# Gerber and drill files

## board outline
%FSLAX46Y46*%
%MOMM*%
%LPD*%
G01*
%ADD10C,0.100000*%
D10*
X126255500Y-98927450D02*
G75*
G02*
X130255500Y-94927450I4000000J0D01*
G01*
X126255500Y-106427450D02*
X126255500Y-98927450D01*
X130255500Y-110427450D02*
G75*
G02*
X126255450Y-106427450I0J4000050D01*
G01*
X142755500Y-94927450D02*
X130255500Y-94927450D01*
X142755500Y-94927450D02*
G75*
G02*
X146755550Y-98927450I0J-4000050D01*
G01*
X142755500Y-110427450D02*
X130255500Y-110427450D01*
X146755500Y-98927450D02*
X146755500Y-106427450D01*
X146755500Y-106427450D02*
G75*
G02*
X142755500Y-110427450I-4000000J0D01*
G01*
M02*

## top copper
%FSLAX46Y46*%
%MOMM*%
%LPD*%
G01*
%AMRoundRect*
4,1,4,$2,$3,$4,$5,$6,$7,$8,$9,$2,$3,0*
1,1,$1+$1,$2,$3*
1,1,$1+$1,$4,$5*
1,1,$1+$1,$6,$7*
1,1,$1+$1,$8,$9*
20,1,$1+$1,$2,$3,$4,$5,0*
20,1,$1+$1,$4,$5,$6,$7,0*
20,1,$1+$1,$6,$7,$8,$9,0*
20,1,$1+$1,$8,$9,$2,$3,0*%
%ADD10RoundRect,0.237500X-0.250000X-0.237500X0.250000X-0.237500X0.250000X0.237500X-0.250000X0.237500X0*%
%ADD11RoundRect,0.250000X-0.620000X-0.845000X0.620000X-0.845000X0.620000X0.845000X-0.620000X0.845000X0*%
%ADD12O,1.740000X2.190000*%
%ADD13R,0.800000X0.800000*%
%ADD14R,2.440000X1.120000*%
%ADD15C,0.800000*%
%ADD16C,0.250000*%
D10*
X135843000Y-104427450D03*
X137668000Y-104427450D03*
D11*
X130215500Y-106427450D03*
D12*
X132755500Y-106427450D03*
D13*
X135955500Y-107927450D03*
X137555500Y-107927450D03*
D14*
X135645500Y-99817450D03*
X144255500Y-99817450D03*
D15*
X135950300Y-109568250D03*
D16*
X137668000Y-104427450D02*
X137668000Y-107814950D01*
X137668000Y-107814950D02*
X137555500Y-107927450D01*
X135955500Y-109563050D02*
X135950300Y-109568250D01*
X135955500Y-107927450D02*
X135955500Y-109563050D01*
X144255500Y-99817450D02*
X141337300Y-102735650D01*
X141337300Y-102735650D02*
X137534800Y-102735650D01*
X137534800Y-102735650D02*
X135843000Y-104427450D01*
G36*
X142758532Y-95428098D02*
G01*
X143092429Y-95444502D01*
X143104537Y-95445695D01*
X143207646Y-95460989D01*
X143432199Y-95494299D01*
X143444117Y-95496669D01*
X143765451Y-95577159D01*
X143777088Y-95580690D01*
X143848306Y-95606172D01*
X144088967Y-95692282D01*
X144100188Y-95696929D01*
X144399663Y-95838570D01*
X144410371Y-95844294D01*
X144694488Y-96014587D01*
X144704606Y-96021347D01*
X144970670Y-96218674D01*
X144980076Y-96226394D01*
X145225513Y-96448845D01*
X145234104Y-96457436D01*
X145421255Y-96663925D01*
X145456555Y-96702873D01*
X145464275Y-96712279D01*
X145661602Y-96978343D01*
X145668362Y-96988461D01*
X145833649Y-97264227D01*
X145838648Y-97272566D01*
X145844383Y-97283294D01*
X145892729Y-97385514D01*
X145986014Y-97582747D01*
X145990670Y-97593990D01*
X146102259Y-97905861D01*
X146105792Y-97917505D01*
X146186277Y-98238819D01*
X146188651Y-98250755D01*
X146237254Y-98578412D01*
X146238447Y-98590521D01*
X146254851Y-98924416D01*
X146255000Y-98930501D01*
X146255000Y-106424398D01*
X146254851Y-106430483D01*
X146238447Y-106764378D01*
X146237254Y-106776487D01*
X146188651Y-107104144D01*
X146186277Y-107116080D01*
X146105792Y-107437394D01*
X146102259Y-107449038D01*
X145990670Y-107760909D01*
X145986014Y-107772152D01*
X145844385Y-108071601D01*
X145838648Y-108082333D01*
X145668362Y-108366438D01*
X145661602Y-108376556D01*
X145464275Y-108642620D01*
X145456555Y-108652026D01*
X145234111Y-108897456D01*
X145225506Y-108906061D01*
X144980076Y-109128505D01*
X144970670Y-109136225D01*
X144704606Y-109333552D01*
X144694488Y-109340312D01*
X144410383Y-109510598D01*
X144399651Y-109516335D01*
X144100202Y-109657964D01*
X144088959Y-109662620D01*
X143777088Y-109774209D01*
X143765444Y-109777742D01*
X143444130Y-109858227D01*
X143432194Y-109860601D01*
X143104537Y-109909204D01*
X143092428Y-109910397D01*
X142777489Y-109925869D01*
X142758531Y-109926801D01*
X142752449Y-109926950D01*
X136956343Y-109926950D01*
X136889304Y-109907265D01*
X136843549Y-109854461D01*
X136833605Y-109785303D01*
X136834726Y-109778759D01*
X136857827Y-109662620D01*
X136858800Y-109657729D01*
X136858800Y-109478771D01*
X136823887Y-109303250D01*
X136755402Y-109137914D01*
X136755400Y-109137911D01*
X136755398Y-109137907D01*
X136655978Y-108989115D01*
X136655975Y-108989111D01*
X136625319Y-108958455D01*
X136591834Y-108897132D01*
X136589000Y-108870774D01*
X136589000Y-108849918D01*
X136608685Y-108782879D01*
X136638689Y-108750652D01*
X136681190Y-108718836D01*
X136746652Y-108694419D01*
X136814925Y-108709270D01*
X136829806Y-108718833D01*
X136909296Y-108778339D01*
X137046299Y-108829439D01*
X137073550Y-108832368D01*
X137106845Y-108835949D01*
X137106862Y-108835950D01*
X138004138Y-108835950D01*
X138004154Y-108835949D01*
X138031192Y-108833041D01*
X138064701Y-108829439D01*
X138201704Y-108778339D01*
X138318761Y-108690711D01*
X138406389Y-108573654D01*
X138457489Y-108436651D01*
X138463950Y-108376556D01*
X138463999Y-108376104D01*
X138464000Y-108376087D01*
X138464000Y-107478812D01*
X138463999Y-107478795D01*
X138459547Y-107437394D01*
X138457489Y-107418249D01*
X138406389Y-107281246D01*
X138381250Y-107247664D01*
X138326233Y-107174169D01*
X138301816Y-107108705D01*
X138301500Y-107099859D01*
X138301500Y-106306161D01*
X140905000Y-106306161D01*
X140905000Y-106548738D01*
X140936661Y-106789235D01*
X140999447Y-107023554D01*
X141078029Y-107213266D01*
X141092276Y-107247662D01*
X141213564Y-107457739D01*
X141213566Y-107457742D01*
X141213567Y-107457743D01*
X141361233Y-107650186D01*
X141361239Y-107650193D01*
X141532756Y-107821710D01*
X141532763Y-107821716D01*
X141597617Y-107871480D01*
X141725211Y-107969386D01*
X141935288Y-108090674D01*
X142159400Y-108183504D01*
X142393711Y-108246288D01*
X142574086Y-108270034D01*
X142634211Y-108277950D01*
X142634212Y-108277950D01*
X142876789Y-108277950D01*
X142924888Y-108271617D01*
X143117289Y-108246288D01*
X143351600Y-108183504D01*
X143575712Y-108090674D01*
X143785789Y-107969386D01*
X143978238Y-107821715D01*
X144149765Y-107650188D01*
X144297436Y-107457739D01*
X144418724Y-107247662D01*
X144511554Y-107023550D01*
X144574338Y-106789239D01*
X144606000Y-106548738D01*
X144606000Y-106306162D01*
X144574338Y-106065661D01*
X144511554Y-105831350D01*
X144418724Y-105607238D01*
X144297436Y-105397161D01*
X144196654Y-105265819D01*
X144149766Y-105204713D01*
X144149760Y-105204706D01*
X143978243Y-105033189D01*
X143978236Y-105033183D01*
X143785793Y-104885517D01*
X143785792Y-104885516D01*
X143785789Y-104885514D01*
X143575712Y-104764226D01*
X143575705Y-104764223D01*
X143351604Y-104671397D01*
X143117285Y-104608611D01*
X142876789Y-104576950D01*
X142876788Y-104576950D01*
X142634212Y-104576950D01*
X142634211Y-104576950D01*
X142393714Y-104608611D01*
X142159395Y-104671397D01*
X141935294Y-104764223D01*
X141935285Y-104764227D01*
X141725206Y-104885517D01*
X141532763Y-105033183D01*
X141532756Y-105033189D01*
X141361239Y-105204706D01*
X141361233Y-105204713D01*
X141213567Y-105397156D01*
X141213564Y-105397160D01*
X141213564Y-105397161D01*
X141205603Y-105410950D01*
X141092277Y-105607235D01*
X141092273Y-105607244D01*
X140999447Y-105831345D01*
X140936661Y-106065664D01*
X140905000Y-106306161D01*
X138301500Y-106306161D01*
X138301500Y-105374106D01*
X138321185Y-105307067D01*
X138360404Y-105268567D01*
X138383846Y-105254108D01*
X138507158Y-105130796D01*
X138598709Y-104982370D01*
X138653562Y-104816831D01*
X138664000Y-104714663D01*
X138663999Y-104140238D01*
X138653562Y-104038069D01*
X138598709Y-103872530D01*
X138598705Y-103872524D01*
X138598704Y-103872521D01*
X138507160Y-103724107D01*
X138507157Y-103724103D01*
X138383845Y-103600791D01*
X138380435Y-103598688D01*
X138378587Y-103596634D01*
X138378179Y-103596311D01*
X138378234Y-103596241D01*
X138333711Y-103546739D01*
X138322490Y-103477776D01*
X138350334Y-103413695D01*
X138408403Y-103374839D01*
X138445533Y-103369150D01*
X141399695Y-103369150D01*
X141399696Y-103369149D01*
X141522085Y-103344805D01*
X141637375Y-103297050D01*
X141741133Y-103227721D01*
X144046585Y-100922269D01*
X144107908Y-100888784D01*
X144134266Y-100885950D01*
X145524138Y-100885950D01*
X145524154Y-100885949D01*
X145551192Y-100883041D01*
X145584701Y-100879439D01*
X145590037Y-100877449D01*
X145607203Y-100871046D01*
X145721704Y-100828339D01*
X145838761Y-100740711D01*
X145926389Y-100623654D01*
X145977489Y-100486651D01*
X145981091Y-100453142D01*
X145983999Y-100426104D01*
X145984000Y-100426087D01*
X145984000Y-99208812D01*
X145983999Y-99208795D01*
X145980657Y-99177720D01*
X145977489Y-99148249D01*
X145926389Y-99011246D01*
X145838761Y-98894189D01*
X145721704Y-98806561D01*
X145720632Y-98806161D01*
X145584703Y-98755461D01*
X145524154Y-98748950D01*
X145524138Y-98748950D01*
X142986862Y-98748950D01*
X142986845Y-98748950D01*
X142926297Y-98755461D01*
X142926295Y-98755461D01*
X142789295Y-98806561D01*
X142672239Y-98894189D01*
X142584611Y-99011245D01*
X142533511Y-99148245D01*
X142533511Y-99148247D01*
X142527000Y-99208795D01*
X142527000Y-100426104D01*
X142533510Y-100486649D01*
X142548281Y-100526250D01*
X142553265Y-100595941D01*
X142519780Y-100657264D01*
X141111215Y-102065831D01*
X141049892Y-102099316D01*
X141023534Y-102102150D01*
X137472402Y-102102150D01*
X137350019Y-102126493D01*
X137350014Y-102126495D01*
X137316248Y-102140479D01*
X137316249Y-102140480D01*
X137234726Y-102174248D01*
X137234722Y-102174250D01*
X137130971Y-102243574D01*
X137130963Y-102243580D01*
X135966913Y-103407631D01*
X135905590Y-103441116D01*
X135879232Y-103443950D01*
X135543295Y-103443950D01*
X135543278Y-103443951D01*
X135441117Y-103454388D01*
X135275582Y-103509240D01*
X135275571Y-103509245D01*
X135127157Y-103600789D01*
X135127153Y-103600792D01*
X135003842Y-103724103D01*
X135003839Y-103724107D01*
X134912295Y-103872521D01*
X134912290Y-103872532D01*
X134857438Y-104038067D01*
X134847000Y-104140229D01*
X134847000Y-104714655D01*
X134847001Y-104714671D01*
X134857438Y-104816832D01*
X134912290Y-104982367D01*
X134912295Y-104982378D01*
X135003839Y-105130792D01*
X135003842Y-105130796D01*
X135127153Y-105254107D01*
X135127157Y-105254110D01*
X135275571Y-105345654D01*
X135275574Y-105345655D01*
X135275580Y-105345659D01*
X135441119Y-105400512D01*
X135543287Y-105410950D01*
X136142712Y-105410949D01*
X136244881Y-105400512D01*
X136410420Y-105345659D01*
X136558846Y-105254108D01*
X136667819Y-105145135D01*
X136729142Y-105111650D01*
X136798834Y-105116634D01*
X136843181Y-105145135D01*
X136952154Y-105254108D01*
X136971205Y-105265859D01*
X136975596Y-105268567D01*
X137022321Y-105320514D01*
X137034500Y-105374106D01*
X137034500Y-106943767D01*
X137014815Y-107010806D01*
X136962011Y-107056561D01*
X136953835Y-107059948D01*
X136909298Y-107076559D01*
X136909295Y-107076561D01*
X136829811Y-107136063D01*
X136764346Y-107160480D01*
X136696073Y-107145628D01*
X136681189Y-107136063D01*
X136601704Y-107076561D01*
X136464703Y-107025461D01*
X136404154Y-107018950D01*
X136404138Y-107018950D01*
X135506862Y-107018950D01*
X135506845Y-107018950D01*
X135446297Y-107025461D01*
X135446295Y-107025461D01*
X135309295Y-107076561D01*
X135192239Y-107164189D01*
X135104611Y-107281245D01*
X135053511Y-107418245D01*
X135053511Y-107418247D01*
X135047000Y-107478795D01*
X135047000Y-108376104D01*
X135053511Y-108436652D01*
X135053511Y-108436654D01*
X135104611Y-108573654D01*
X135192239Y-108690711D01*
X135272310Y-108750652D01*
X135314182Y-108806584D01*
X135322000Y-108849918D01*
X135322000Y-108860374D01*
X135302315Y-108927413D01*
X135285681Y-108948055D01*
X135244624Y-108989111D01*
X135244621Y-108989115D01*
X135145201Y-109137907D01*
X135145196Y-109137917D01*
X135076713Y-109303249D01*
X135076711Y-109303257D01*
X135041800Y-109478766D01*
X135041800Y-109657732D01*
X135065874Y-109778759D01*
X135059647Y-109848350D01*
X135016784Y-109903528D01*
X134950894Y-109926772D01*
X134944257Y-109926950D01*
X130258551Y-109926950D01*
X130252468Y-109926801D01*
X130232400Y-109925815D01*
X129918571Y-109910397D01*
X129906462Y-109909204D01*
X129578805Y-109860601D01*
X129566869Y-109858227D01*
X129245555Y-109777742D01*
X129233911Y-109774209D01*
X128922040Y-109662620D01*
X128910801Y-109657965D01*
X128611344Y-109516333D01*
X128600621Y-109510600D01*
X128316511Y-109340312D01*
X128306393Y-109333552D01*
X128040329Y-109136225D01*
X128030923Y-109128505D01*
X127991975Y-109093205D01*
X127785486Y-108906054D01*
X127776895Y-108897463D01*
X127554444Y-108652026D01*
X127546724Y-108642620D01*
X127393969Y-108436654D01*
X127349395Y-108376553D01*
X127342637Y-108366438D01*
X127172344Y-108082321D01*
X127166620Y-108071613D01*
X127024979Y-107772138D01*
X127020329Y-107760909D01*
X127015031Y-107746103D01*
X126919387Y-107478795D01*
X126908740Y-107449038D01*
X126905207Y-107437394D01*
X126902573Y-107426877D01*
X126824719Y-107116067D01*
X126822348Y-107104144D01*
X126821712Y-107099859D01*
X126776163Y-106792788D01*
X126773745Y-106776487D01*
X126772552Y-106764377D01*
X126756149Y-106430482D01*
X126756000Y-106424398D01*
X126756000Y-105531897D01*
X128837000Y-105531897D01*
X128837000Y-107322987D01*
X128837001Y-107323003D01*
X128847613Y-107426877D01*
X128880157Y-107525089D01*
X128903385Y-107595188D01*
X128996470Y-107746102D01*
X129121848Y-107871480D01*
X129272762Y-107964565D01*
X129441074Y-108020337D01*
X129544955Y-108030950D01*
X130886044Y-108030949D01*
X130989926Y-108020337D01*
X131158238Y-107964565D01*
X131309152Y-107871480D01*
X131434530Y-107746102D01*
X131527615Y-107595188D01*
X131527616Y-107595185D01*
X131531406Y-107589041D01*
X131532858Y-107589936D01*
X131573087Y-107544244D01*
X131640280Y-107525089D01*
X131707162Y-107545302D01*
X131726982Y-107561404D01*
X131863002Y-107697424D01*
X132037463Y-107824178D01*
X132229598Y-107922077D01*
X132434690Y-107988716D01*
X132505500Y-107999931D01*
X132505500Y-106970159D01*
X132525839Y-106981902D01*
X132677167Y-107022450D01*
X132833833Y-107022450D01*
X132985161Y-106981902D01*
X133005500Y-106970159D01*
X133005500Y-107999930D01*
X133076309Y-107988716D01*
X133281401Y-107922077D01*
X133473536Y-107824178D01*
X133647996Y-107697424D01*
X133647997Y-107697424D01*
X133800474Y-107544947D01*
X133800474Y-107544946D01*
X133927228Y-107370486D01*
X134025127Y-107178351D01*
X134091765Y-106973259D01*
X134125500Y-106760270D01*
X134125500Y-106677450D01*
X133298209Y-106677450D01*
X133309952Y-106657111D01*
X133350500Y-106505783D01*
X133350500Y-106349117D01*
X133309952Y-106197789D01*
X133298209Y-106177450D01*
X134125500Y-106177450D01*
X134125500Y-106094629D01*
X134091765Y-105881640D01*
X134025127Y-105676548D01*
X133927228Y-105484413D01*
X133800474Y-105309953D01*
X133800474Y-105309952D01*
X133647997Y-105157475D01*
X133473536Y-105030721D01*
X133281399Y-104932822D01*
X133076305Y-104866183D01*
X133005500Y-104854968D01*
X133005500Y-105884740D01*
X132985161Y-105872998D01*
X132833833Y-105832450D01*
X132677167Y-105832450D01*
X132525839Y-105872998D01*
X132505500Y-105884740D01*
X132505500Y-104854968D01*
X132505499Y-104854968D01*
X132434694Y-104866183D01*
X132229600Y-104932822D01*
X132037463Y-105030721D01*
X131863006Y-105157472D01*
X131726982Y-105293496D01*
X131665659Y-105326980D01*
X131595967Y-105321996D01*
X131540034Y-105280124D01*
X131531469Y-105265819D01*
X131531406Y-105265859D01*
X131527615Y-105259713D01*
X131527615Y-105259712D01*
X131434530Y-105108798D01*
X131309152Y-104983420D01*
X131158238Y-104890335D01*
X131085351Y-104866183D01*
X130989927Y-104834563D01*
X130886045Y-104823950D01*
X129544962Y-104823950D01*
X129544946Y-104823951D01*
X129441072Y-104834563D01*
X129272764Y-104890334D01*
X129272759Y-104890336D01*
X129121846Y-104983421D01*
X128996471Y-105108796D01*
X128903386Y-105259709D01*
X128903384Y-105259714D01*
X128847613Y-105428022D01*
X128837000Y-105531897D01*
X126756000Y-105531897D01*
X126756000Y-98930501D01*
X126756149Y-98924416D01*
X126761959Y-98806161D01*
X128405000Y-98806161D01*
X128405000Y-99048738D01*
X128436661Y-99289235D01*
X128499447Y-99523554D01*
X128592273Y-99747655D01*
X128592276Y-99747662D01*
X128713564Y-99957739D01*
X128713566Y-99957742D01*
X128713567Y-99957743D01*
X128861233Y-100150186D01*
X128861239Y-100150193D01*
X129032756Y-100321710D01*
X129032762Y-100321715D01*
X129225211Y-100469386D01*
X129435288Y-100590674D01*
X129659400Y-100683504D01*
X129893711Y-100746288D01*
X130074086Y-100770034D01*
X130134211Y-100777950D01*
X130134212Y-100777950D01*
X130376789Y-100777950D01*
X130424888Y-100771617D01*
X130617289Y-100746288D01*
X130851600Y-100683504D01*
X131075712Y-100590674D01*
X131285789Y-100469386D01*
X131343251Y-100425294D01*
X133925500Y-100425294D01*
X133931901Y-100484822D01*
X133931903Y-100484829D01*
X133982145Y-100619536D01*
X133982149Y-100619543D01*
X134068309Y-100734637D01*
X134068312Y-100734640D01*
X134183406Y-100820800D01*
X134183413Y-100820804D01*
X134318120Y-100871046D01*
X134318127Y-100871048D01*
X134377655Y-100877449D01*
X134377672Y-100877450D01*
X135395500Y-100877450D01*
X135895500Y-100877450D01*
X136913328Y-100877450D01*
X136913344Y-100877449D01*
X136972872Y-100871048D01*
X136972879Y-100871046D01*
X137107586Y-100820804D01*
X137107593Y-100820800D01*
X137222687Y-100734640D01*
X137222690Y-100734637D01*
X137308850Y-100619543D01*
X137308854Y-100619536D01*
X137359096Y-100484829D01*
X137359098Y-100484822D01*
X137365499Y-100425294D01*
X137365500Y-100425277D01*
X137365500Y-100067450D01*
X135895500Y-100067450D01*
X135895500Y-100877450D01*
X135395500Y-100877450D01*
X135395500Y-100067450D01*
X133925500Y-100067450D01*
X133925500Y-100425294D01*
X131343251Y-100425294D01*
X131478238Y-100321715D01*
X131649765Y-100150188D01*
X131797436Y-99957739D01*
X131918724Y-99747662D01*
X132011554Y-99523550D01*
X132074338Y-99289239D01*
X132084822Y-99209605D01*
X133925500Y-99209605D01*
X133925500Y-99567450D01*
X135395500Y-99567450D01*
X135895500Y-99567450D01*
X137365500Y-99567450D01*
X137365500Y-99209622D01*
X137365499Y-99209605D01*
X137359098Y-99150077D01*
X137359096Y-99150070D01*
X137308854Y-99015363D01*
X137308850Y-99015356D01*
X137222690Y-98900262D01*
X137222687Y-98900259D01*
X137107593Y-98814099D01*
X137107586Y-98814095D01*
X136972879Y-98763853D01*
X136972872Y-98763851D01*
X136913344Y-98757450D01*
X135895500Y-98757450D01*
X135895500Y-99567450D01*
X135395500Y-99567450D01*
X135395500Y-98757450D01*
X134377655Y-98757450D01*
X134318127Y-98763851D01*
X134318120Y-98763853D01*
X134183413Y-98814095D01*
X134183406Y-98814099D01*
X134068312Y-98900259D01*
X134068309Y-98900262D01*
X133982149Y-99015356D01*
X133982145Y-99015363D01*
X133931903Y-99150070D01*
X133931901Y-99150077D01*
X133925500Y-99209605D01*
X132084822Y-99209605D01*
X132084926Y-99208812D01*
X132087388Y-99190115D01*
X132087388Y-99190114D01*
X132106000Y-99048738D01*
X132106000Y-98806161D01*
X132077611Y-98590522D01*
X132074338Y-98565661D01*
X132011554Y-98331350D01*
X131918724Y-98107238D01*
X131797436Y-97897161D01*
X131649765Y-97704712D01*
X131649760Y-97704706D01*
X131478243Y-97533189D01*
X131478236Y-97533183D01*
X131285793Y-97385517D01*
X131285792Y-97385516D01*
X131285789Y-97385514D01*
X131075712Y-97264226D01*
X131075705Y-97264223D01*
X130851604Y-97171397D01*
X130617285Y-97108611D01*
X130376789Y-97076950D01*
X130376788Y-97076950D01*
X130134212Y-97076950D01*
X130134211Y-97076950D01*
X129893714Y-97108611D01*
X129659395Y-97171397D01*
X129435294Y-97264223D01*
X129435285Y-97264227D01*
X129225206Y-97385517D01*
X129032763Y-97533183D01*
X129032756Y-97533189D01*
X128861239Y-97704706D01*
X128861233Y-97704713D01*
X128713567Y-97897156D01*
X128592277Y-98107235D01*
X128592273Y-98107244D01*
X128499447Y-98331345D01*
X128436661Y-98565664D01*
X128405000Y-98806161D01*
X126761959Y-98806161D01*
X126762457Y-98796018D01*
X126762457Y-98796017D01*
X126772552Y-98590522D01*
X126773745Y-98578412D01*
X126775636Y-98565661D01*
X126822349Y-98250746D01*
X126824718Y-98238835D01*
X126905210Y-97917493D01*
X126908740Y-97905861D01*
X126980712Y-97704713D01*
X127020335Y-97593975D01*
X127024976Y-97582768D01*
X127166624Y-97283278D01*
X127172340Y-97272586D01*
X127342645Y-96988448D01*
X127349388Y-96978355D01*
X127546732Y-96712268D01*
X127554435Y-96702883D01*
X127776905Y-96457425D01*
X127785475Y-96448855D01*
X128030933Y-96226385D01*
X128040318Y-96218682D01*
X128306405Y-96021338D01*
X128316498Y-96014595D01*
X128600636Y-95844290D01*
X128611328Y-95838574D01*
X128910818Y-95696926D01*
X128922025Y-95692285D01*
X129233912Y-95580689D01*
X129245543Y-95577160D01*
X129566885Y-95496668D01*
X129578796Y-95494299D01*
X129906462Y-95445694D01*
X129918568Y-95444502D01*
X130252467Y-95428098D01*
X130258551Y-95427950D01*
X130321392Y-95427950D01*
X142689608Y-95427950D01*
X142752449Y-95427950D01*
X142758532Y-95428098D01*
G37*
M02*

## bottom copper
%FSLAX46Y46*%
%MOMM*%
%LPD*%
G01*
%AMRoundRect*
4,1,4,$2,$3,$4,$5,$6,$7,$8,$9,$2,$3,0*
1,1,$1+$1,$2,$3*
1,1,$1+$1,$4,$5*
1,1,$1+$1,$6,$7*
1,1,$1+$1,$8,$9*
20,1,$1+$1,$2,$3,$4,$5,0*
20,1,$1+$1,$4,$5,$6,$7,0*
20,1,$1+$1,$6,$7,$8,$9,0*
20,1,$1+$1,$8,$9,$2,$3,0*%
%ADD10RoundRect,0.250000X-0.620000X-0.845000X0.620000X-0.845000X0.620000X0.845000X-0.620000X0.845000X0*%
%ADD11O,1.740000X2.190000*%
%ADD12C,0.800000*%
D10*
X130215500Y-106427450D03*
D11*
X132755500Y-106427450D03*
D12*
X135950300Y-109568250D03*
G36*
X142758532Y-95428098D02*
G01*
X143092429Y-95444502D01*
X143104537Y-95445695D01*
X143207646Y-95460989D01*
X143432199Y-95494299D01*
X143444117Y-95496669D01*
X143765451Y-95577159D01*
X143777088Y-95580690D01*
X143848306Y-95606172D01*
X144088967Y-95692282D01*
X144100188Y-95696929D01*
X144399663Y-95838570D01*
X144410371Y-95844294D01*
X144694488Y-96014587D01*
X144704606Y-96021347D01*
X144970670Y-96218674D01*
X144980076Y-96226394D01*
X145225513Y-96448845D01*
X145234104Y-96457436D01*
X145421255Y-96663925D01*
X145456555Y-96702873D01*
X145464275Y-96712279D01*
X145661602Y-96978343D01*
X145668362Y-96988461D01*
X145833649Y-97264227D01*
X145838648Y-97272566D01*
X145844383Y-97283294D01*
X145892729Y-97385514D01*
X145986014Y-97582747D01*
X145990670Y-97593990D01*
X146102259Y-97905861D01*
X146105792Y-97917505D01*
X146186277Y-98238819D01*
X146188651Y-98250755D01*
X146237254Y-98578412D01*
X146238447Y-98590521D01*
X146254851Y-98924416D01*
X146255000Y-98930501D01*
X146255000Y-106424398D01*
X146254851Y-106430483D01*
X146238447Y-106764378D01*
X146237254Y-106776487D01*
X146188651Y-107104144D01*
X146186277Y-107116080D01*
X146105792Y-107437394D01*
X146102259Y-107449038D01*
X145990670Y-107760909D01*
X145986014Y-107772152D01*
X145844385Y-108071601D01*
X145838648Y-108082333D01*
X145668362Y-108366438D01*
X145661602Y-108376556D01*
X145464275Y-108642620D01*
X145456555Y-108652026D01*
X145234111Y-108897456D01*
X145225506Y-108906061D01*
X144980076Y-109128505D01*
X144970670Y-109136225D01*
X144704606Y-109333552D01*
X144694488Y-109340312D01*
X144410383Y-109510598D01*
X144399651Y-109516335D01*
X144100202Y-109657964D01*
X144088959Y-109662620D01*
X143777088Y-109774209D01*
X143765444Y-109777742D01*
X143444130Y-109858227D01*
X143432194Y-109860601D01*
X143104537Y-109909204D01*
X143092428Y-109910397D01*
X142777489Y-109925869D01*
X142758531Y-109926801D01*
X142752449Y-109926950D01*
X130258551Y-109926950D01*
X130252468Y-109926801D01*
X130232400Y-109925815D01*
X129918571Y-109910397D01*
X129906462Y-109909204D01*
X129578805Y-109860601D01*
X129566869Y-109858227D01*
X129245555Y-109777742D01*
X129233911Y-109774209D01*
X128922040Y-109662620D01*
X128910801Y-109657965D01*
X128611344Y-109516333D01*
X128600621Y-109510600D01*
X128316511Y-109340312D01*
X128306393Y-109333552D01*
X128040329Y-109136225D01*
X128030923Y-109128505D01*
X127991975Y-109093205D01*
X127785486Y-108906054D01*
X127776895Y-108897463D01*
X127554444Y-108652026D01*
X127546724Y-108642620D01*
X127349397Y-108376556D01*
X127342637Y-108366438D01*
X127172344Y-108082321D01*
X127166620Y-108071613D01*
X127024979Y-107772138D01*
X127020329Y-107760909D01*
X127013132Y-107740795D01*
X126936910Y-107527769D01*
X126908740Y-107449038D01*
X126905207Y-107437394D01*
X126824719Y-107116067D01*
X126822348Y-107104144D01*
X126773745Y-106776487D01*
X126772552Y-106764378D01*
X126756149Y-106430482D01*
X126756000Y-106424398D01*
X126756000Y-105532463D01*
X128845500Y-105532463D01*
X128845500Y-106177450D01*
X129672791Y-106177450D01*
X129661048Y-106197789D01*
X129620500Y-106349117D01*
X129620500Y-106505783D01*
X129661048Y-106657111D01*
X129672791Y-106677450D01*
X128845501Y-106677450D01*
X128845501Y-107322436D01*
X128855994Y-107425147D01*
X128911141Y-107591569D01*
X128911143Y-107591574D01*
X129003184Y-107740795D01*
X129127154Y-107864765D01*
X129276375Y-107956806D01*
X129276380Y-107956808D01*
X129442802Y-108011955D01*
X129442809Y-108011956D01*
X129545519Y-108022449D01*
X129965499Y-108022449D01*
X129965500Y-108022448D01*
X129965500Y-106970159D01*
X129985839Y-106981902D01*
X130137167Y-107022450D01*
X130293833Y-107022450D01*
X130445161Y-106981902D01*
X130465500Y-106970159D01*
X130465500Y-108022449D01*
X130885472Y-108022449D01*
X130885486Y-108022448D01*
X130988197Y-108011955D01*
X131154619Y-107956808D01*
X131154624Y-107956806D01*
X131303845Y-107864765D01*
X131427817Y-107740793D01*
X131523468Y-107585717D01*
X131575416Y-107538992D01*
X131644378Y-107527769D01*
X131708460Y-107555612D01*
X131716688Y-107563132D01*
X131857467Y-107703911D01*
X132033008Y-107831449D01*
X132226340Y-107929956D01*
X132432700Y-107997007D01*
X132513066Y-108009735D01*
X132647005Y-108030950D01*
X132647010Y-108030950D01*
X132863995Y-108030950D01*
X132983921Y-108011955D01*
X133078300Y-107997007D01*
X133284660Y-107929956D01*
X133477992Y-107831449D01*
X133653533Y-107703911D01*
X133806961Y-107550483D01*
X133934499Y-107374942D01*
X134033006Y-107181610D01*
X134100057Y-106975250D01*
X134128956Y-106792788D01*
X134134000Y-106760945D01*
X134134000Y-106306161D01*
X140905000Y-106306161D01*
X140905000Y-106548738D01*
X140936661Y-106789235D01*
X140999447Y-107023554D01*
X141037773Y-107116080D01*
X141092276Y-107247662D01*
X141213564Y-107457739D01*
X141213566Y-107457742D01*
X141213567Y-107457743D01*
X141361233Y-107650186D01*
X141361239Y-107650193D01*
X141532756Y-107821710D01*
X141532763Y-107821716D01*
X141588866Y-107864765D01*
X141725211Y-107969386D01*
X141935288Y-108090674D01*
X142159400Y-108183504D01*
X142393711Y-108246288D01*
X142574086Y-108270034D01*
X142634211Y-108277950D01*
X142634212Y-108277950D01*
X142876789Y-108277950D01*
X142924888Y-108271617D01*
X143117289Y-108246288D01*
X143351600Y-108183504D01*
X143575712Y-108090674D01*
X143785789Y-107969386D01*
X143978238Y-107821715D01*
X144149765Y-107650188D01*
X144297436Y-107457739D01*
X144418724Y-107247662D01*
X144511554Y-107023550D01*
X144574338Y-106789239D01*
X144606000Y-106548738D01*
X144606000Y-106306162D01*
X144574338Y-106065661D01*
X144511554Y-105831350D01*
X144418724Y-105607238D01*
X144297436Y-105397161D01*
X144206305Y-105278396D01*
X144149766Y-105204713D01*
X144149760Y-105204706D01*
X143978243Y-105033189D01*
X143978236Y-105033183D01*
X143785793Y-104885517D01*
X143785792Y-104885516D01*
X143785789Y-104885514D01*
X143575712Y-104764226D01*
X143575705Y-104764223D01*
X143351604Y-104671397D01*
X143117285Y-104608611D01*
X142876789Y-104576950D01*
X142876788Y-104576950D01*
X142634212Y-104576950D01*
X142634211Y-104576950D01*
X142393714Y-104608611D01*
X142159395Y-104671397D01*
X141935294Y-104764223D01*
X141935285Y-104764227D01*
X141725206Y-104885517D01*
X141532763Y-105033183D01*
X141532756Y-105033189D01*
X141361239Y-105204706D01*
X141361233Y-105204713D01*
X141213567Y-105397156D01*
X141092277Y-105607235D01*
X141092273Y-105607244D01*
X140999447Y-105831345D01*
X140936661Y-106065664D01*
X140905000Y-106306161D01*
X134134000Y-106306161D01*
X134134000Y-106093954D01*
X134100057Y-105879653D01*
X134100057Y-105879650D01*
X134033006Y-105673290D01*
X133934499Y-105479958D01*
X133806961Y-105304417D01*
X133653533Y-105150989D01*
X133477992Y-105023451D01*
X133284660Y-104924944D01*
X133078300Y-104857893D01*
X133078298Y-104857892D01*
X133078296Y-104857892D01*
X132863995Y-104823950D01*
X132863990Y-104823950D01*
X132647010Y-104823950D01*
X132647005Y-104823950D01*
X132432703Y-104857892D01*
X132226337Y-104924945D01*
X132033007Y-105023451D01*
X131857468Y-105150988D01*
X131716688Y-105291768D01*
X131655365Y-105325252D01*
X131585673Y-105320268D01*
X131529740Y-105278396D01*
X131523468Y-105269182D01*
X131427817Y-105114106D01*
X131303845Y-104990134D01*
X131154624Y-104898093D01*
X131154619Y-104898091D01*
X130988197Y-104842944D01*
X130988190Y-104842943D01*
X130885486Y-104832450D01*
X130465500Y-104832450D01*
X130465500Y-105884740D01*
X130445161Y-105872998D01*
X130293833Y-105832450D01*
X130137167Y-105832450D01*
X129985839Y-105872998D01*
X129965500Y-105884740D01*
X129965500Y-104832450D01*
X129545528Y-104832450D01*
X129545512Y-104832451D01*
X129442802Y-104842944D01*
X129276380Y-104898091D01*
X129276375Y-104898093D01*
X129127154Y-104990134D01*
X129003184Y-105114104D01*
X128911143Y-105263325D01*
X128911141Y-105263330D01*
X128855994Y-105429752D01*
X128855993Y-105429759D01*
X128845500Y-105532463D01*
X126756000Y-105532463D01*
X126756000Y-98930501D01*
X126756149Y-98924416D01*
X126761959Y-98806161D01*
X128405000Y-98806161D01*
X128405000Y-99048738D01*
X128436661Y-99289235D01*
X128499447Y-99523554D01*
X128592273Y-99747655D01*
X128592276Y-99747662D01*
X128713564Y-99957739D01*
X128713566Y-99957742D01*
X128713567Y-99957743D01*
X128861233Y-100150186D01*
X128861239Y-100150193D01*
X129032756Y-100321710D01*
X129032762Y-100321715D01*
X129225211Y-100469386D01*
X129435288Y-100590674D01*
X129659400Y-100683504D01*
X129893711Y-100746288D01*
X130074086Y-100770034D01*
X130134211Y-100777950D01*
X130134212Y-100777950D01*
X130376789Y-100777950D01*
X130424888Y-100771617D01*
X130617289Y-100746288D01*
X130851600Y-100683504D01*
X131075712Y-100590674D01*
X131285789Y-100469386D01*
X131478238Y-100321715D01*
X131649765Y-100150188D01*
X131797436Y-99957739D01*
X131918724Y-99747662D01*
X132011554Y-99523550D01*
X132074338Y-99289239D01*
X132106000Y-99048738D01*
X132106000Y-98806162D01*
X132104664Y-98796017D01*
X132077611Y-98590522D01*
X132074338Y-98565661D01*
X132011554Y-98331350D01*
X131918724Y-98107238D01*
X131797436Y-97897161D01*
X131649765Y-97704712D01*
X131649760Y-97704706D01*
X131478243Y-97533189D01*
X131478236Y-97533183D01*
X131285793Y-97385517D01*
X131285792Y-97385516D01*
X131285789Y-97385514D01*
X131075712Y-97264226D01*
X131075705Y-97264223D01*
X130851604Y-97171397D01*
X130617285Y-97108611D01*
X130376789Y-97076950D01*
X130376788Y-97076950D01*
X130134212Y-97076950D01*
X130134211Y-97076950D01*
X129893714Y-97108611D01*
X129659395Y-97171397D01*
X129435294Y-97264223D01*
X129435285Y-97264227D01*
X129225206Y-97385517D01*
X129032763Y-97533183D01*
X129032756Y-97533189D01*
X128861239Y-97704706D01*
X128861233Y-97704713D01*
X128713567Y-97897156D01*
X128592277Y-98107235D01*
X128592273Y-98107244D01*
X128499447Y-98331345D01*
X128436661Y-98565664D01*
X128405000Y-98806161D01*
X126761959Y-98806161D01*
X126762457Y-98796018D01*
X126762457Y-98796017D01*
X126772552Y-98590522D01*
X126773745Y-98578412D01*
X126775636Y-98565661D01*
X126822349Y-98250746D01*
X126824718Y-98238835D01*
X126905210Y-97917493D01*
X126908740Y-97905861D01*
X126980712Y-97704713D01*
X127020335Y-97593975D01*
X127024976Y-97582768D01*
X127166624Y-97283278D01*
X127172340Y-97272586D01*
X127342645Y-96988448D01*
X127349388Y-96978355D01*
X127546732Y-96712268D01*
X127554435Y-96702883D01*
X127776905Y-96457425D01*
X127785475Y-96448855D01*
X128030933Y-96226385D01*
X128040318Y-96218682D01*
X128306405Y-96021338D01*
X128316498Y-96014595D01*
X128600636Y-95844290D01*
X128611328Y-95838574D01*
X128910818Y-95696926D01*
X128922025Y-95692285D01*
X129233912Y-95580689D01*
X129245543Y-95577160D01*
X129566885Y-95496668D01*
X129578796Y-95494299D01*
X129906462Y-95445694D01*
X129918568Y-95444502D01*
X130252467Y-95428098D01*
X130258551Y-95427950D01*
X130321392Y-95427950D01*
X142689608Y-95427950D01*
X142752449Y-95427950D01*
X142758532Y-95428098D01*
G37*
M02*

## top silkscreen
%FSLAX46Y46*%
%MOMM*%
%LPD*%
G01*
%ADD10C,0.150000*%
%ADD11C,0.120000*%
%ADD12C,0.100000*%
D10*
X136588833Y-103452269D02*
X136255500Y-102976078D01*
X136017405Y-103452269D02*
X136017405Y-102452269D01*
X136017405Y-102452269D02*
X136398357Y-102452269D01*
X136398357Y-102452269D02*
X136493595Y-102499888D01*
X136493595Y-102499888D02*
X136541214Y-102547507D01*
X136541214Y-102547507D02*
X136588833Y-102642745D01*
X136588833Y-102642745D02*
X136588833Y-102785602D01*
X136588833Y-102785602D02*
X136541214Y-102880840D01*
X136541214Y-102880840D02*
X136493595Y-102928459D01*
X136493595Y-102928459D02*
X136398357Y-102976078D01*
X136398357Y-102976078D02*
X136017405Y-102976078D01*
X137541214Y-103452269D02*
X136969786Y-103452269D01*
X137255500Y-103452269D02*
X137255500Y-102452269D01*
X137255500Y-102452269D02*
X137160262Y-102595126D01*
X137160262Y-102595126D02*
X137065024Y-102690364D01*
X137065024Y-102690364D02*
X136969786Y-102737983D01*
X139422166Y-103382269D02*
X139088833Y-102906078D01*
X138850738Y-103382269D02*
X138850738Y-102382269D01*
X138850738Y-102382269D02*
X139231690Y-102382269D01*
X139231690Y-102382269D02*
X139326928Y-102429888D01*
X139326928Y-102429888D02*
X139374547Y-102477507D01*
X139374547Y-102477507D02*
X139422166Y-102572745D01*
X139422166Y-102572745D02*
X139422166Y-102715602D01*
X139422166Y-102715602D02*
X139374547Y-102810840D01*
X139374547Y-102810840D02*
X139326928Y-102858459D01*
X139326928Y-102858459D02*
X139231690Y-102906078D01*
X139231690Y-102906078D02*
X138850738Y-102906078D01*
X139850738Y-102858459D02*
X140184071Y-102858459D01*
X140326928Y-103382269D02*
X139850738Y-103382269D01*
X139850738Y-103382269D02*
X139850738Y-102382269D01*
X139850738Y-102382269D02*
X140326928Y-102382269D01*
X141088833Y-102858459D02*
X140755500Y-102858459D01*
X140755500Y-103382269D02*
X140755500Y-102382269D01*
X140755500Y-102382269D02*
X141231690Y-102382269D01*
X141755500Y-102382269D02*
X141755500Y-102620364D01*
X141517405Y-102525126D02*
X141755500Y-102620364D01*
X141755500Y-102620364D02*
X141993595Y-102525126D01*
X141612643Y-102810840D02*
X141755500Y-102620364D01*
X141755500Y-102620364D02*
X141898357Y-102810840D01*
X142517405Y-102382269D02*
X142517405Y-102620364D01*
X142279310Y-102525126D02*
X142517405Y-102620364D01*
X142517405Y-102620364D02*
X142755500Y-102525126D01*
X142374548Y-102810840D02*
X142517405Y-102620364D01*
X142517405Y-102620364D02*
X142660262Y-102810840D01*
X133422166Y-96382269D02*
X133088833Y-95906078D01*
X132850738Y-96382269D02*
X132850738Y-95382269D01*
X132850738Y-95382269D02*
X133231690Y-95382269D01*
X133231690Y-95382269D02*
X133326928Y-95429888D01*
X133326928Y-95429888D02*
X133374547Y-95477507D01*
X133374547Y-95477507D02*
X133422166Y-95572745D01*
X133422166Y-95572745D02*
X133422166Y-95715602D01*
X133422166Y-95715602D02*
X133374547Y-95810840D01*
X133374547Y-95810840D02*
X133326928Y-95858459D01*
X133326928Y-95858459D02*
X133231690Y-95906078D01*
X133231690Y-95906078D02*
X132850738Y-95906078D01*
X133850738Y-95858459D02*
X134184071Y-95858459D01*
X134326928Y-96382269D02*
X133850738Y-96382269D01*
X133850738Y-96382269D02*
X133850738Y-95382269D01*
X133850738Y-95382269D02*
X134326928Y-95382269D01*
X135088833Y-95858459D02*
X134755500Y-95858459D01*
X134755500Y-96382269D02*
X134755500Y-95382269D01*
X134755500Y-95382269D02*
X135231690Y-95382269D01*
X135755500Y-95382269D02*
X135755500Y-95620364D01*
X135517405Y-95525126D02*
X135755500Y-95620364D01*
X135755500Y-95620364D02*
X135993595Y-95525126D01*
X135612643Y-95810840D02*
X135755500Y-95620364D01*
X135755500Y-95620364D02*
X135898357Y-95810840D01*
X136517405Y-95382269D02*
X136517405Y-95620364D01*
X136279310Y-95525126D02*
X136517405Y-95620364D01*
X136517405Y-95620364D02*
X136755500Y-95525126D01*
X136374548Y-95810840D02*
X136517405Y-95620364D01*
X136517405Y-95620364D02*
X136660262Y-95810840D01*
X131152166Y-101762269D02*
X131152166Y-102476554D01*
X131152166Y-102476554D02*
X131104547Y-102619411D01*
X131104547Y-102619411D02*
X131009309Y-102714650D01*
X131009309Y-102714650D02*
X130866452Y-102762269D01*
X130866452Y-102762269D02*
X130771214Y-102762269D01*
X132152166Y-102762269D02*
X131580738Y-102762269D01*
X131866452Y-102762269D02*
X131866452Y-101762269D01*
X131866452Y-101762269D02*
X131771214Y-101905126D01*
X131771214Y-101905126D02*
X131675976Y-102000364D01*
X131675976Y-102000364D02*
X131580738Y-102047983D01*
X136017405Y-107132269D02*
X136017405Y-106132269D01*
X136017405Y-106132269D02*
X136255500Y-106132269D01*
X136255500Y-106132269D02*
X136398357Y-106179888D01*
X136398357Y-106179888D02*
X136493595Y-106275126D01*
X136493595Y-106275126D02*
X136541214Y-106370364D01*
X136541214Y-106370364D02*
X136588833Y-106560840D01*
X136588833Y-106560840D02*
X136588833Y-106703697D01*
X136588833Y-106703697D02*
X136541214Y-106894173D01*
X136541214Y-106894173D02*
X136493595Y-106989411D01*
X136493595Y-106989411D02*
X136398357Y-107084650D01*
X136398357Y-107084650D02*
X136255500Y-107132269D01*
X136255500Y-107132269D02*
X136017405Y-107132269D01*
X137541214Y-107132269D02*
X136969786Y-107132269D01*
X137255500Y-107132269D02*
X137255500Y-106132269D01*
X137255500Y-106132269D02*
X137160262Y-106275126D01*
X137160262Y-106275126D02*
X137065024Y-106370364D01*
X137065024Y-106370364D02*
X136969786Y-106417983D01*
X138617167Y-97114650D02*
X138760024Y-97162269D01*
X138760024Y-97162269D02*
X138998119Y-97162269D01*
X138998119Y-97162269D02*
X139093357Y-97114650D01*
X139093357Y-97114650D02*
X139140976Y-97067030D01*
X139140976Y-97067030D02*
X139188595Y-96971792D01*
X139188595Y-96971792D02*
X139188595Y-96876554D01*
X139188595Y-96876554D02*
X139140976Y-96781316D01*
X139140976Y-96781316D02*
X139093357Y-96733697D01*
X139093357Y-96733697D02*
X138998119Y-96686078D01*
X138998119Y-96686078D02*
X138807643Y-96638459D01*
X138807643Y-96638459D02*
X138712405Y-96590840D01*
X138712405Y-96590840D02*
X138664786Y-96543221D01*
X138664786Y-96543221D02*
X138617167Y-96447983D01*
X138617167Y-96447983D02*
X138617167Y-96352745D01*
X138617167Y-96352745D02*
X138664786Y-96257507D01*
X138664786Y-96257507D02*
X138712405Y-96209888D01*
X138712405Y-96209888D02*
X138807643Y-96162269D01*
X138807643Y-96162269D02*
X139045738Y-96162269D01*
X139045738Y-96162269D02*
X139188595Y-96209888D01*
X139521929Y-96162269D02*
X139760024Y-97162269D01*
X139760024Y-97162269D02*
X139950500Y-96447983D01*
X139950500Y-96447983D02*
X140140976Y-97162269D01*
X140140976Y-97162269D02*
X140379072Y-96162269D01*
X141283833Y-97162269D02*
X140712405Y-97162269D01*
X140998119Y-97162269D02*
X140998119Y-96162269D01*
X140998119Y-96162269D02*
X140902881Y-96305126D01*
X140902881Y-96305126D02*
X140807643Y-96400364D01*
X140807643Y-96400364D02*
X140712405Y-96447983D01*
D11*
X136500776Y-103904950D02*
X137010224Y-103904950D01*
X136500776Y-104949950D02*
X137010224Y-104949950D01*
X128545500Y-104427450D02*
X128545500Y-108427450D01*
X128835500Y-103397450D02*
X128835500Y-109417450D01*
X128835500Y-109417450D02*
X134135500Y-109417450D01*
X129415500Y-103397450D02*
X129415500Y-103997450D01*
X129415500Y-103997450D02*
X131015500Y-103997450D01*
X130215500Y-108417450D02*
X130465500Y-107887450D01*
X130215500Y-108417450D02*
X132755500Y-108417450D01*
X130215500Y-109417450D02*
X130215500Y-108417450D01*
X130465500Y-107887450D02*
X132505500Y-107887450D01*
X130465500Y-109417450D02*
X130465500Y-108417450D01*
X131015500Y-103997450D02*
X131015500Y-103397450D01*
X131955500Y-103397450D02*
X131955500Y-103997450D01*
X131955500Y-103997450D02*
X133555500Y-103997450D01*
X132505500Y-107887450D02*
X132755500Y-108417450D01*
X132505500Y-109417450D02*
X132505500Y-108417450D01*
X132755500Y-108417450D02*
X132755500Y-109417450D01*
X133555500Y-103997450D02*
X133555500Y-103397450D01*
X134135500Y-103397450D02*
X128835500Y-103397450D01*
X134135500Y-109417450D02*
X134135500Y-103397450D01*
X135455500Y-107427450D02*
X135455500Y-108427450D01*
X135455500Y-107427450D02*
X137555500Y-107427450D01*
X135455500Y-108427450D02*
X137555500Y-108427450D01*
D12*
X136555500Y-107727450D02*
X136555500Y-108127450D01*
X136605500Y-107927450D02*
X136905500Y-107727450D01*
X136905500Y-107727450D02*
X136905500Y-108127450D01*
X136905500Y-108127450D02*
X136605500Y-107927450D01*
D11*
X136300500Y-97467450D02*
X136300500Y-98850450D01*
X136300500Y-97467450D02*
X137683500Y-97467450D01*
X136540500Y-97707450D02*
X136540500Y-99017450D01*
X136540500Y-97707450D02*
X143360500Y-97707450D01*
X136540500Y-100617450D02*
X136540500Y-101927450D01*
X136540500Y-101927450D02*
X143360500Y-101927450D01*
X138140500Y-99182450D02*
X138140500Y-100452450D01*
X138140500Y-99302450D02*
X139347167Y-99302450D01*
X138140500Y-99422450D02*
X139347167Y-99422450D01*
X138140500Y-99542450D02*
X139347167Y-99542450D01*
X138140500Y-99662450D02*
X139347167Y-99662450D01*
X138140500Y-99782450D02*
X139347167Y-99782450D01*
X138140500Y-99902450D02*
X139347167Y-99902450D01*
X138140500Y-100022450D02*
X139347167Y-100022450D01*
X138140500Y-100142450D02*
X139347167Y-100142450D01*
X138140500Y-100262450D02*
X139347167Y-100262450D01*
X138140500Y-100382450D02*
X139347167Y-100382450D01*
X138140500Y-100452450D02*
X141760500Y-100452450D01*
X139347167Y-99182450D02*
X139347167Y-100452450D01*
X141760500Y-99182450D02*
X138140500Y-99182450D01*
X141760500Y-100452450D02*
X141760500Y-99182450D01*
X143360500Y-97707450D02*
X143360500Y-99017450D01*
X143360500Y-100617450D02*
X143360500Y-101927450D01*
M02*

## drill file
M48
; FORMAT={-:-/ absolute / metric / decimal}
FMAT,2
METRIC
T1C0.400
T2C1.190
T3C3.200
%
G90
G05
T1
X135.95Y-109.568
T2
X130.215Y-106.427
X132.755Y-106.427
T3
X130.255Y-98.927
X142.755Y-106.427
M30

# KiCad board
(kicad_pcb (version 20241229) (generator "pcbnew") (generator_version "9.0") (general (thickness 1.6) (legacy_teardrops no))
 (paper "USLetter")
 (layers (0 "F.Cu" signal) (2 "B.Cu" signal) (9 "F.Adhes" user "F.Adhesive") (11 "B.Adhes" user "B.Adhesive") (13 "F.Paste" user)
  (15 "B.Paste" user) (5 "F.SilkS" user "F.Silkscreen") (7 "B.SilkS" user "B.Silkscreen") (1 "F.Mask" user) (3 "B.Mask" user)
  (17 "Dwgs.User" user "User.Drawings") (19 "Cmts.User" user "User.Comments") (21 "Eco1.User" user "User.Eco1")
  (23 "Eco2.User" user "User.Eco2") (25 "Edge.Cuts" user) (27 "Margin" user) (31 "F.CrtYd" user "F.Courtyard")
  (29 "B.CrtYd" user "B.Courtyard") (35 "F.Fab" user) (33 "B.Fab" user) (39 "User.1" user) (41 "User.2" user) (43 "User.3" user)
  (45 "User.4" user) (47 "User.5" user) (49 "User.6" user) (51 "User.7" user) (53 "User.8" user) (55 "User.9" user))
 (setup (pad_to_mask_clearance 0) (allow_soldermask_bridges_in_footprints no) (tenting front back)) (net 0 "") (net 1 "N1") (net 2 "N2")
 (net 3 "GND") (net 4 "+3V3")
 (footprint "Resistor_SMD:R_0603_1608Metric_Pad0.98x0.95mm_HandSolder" (layer "F.Cu") (at 136.7555 104.42745)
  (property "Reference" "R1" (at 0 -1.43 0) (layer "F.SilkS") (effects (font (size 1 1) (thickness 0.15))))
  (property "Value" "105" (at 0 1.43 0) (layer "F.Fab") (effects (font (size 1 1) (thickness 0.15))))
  (fp_line (start -0.254724 -0.5225) (end 0.254724 -0.5225) (stroke (width 0.12) (type solid)) (layer "F.SilkS"))
  (fp_line (start -0.254724 0.5225) (end 0.254724 0.5225) (stroke (width 0.12) (type solid)) (layer "F.SilkS"))
  (pad "1" smd roundrect (at -0.9125 0) (size 0.975 0.95) (layers "F.Cu" "F.Mask" "F.Paste") (roundrect_rratio 0.25) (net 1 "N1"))
  (pad "2" smd roundrect (at 0.9125 0) (size 0.975 0.95) (layers "F.Cu" "F.Mask" "F.Paste") (roundrect_rratio 0.25) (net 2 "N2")))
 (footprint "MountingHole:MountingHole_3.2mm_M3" (layer "F.Cu") (at 142.7555 106.42745)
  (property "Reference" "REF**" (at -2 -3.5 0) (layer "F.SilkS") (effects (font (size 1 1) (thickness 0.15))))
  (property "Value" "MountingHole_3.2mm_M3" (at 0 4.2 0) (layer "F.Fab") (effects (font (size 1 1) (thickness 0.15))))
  (pad "" np_thru_hole circle (at 0 0) (size 3.2 3.2) (drill 3.2) (layers "*.Cu" "*.Mask")))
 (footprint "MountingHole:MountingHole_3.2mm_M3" (layer "F.Cu") (at 130.2555 98.92745)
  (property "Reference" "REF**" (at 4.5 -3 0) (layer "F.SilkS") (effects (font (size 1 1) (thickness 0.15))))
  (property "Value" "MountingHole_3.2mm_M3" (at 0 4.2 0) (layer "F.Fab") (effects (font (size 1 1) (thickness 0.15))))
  (pad "" np_thru_hole circle (at 0 0) (size 3.2 3.2) (drill 3.2) (layers "*.Cu" "*.Mask")))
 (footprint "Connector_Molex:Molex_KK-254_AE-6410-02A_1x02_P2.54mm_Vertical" (layer "F.Cu") (at 130.2155 106.42745)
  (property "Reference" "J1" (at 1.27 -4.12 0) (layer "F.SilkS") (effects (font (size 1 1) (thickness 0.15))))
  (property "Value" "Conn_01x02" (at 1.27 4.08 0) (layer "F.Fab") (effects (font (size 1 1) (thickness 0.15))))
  (fp_line (start -1.67 -2) (end -1.67 2) (stroke (width 0.12) (type solid)) (layer "F.SilkS"))
  (fp_line (start -1.38 -3.03) (end -1.38 2.99) (stroke (width 0.12) (type solid)) (layer "F.SilkS"))
  (fp_line (start -1.38 2.99) (end 3.92 2.99) (stroke (width 0.12) (type solid)) (layer "F.SilkS"))
  (fp_line (start -0.8 -3.03) (end -0.8 -2.43) (stroke (width 0.12) (type solid)) (layer "F.SilkS"))
  (fp_line (start -0.8 -2.43) (end 0.8 -2.43) (stroke (width 0.12) (type solid)) (layer "F.SilkS"))
  (fp_line (start 0 1.99) (end 0.25 1.46) (stroke (width 0.12) (type solid)) (layer "F.SilkS"))
  (fp_line (start 0 1.99) (end 2.54 1.99) (stroke (width 0.12) (type solid)) (layer "F.SilkS"))
  (fp_line (start 0 2.99) (end 0 1.99) (stroke (width 0.12) (type solid)) (layer "F.SilkS"))
  (fp_line (start 0.25 1.46) (end 2.29 1.46) (stroke (width 0.12) (type solid)) (layer "F.SilkS"))
  (fp_line (start 0.25 2.99) (end 0.25 1.99) (stroke (width 0.12) (type solid)) (layer "F.SilkS"))
  (fp_line (start 0.8 -2.43) (end 0.8 -3.03) (stroke (width 0.12) (type solid)) (layer "F.SilkS"))
  (fp_line (start 1.74 -3.03) (end 1.74 -2.43) (stroke (width 0.12) (type solid)) (layer "F.SilkS"))
  (fp_line (start 1.74 -2.43) (end 3.34 -2.43) (stroke (width 0.12) (type solid)) (layer "F.SilkS"))
  (fp_line (start 2.29 1.46) (end 2.54 1.99) (stroke (width 0.12) (type solid)) (layer "F.SilkS"))
  (fp_line (start 2.29 2.99) (end 2.29 1.99) (stroke (width 0.12) (type solid)) (layer "F.SilkS"))
  (fp_line (start 2.54 1.99) (end 2.54 2.99) (stroke (width 0.12) (type solid)) (layer "F.SilkS"))
  (fp_line (start 3.34 -2.43) (end 3.34 -3.03) (stroke (width 0.12) (type solid)) (layer "F.SilkS"))
  (fp_line (start 3.92 -3.03) (end -1.38 -3.03) (stroke (width 0.12) (type solid)) (layer "F.SilkS"))
  (fp_line (start 3.92 2.99) (end 3.92 -3.03) (stroke (width 0.12) (type solid)) (layer "F.SilkS"))
  (pad "1" thru_hole roundrect (at 0 0) (size 1.74 2.19) (drill 1.19) (layers "*.Cu" "*.Mask") (remove_unused_layers no)
   (roundrect_rratio 0.143678) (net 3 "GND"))
  (pad "2" thru_hole oval (at 2.54 0) (size 1.74 2.19) (drill 1.19) (layers "*.Cu" "*.Mask") (remove_unused_layers no) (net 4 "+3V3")))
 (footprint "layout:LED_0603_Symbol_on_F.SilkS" (layer "F.Cu") (at 136.7555 107.92745)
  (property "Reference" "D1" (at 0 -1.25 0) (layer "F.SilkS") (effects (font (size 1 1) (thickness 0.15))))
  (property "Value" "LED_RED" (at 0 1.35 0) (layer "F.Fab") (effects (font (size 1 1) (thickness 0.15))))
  (fp_line (start -1.3 -0.5) (end -1.3 0.5) (stroke (width 0.12) (type solid)) (layer "F.SilkS"))
  (fp_line (start -1.3 -0.5) (end 0.8 -0.5) (stroke (width 0.12) (type solid)) (layer "F.SilkS"))
  (fp_line (start -1.3 0.5) (end 0.8 0.5) (stroke (width 0.12) (type solid)) (layer "F.SilkS"))
  (fp_line (start -0.2 -0.2) (end -0.2 0.2) (stroke (width 0.1) (type solid)) (layer "F.SilkS"))
  (fp_line (start -0.15 0) (end 0.15 -0.2) (stroke (width 0.1) (type solid)) (layer "F.SilkS"))
  (fp_line (start 0.15 -0.2) (end 0.15 0.2) (stroke (width 0.1) (type solid)) (layer "F.SilkS"))
  (fp_line (start 0.15 0.2) (end -0.15 0) (stroke (width 0.1) (type solid)) (layer "F.SilkS"))
  (pad "1" smd rect (at -0.8 0 180) (size 0.8 0.8) (layers "F.Cu" "F.Mask" "F.Paste") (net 3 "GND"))
  (pad "2" smd rect (at 0.8 0 180) (size 0.8 0.8) (layers "F.Cu" "F.Mask" "F.Paste") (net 2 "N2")))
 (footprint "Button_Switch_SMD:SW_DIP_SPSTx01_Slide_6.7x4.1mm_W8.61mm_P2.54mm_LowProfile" (layer "F.Cu") (at 139.9505 99.81745)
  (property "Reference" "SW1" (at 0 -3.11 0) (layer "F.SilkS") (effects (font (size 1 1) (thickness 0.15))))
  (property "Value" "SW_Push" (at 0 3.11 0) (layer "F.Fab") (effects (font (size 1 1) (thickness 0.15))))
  (fp_line (start -3.65 -2.35) (end -3.65 -0.967) (stroke (width 0.12) (type solid)) (layer "F.SilkS"))
  (fp_line (start -3.65 -2.35) (end -2.267 -2.35) (stroke (width 0.12) (type solid)) (layer "F.SilkS"))
  (fp_line (start -3.41 -2.11) (end -3.41 -0.8) (stroke (width 0.12) (type solid)) (layer "F.SilkS"))
  (fp_line (start -3.41 -2.11) (end 3.41 -2.11) (stroke (width 0.12) (type solid)) (layer "F.SilkS"))
  (fp_line (start -3.41 0.8) (end -3.41 2.11) (stroke (width 0.12) (type solid)) (layer "F.SilkS"))
  (fp_line (start -3.41 2.11) (end 3.41 2.11) (stroke (width 0.12) (type solid)) (layer "F.SilkS"))
  (fp_line (start -1.81 -0.635) (end -1.81 0.635) (stroke (width 0.12) (type solid)) (layer "F.SilkS"))
  (fp_line (start -1.81 -0.515) (end -0.603333 -0.515) (stroke (width 0.12) (type solid)) (layer "F.SilkS"))
  (fp_line (start -1.81 -0.395) (end -0.603333 -0.395) (stroke (width 0.12) (type solid)) (layer "F.SilkS"))
  (fp_line (start -1.81 -0.275) (end -0.603333 -0.275) (stroke (width 0.12) (type solid)) (layer "F.SilkS"))
  (fp_line (start -1.81 -0.155) (end -0.603333 -0.155) (stroke (width 0.12) (type solid)) (layer "F.SilkS"))
  (fp_line (start -1.81 -0.035) (end -0.603333 -0.035) (stroke (width 0.12) (type solid)) (layer "F.SilkS"))
  (fp_line (start -1.81 0.085) (end -0.603333 0.085) (stroke (width 0.12) (type solid)) (layer "F.SilkS"))
  (fp_line (start -1.81 0.205) (end -0.603333 0.205) (stroke (width 0.12) (type solid)) (layer "F.SilkS"))
  (fp_line (start -1.81 0.325) (end -0.603333 0.325) (stroke (width 0.12) (type solid)) (layer "F.SilkS"))
  (fp_line (start -1.81 0.445) (end -0.603333 0.445) (stroke (width 0.12) (type solid)) (layer "F.SilkS"))
  (fp_line (start -1.81 0.565) (end -0.603333 0.565) (stroke (width 0.12) (type solid)) (layer "F.SilkS"))
  (fp_line (start -1.81 0.635) (end 1.81 0.635) (stroke (width 0.12) (type solid)) (layer "F.SilkS"))
  (fp_line (start -0.603333 -0.635) (end -0.603333 0.635) (stroke (width 0.12) (type solid)) (layer "F.SilkS"))
  (fp_line (start 1.81 -0.635) (end -1.81 -0.635) (stroke (width 0.12) (type solid)) (layer "F.SilkS"))
  (fp_line (start 1.81 0.635) (end 1.81 -0.635) (stroke (width 0.12) (type solid)) (layer "F.SilkS"))
  (fp_line (start 3.41 -2.11) (end 3.41 -0.8) (stroke (width 0.12) (type solid)) (layer "F.SilkS"))
  (fp_line (start 3.41 0.8) (end 3.41 2.11) (stroke (width 0.12) (type solid)) (layer "F.SilkS"))
  (pad "1" smd rect (at -4.305 0) (size 2.44 1.12) (layers "F.Cu" "F.Mask" "F.Paste") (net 4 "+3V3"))
  (pad "2" smd rect (at 4.305 0) (size 2.44 1.12) (layers "F.Cu" "F.Mask" "F.Paste") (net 1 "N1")))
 (gr_arc (start 126.2555 98.92745) (mid 127.427073 96.099023) (end 130.2555 94.92745) (stroke (width 0.1) (type default))
  (layer "Edge.Cuts"))
 (gr_line (start 126.2555 106.42745) (end 126.2555 98.92745) (stroke (width 0.1) (type default)) (layer "Edge.Cuts"))
 (gr_arc (start 130.2555 110.42745) (mid 127.427073 109.255877) (end 126.2555 106.42745) (stroke (width 0.1) (type default))
  (layer "Edge.Cuts"))
 (gr_line (start 142.7555 94.92745) (end 130.2555 94.92745) (stroke (width 0.1) (type default)) (layer "Edge.Cuts"))
 (gr_arc (start 142.7555 94.92745) (mid 145.583927 96.099023) (end 146.7555 98.92745) (stroke (width 0.1) (type default))
  (layer "Edge.Cuts"))
 (gr_line (start 142.7555 110.42745) (end 130.2555 110.42745) (stroke (width 0.1) (type default)) (layer "Edge.Cuts"))
 (gr_line (start 146.7555 98.92745) (end 146.7555 106.42745) (stroke (width 0.1) (type default)) (layer "Edge.Cuts"))
 (gr_arc (start 146.7555 106.42745) (mid 145.583927 109.255877) (end 142.7555 110.42745) (stroke (width 0.1) (type default))
  (layer "Edge.Cuts"))
 (segment (start 137.668 104.42745) (end 137.668 107.81495) (width 0.25) (layer "F.Cu") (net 2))
 (segment (start 137.668 107.81495) (end 137.5555 107.92745) (width 0.25) (layer "F.Cu") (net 2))
 (segment (start 135.9555 109.56305) (end 135.9503 109.56825) (width 0.25) (layer "F.Cu") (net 3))
 (segment (start 135.9555 107.92745) (end 135.9555 109.56305) (width 0.25) (layer "F.Cu") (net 3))
 (via (at 135.9503 109.56825) (size 0.8) (drill 0.4) (layers "F.Cu" "B.Cu") (free yes) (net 3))
 (segment (start 144.2555 99.81745) (end 141.3373 102.73565) (width 0.25) (layer "F.Cu") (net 1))
 (segment (start 141.3373 102.73565) (end 137.5348 102.73565) (width 0.25) (layer "F.Cu") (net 1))
 (segment (start 137.5348 102.73565) (end 135.843 104.42745) (width 0.25) (layer "F.Cu") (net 1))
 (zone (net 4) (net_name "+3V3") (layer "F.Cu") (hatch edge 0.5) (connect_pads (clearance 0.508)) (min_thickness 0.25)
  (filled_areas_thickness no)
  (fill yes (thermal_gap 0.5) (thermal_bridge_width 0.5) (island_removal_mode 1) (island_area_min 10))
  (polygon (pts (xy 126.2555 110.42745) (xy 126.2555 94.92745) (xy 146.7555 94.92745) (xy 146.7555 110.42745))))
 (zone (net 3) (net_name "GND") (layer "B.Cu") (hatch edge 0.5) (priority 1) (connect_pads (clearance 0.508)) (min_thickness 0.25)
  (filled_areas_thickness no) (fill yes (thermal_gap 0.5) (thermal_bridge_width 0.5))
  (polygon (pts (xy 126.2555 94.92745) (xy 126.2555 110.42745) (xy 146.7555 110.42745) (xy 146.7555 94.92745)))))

